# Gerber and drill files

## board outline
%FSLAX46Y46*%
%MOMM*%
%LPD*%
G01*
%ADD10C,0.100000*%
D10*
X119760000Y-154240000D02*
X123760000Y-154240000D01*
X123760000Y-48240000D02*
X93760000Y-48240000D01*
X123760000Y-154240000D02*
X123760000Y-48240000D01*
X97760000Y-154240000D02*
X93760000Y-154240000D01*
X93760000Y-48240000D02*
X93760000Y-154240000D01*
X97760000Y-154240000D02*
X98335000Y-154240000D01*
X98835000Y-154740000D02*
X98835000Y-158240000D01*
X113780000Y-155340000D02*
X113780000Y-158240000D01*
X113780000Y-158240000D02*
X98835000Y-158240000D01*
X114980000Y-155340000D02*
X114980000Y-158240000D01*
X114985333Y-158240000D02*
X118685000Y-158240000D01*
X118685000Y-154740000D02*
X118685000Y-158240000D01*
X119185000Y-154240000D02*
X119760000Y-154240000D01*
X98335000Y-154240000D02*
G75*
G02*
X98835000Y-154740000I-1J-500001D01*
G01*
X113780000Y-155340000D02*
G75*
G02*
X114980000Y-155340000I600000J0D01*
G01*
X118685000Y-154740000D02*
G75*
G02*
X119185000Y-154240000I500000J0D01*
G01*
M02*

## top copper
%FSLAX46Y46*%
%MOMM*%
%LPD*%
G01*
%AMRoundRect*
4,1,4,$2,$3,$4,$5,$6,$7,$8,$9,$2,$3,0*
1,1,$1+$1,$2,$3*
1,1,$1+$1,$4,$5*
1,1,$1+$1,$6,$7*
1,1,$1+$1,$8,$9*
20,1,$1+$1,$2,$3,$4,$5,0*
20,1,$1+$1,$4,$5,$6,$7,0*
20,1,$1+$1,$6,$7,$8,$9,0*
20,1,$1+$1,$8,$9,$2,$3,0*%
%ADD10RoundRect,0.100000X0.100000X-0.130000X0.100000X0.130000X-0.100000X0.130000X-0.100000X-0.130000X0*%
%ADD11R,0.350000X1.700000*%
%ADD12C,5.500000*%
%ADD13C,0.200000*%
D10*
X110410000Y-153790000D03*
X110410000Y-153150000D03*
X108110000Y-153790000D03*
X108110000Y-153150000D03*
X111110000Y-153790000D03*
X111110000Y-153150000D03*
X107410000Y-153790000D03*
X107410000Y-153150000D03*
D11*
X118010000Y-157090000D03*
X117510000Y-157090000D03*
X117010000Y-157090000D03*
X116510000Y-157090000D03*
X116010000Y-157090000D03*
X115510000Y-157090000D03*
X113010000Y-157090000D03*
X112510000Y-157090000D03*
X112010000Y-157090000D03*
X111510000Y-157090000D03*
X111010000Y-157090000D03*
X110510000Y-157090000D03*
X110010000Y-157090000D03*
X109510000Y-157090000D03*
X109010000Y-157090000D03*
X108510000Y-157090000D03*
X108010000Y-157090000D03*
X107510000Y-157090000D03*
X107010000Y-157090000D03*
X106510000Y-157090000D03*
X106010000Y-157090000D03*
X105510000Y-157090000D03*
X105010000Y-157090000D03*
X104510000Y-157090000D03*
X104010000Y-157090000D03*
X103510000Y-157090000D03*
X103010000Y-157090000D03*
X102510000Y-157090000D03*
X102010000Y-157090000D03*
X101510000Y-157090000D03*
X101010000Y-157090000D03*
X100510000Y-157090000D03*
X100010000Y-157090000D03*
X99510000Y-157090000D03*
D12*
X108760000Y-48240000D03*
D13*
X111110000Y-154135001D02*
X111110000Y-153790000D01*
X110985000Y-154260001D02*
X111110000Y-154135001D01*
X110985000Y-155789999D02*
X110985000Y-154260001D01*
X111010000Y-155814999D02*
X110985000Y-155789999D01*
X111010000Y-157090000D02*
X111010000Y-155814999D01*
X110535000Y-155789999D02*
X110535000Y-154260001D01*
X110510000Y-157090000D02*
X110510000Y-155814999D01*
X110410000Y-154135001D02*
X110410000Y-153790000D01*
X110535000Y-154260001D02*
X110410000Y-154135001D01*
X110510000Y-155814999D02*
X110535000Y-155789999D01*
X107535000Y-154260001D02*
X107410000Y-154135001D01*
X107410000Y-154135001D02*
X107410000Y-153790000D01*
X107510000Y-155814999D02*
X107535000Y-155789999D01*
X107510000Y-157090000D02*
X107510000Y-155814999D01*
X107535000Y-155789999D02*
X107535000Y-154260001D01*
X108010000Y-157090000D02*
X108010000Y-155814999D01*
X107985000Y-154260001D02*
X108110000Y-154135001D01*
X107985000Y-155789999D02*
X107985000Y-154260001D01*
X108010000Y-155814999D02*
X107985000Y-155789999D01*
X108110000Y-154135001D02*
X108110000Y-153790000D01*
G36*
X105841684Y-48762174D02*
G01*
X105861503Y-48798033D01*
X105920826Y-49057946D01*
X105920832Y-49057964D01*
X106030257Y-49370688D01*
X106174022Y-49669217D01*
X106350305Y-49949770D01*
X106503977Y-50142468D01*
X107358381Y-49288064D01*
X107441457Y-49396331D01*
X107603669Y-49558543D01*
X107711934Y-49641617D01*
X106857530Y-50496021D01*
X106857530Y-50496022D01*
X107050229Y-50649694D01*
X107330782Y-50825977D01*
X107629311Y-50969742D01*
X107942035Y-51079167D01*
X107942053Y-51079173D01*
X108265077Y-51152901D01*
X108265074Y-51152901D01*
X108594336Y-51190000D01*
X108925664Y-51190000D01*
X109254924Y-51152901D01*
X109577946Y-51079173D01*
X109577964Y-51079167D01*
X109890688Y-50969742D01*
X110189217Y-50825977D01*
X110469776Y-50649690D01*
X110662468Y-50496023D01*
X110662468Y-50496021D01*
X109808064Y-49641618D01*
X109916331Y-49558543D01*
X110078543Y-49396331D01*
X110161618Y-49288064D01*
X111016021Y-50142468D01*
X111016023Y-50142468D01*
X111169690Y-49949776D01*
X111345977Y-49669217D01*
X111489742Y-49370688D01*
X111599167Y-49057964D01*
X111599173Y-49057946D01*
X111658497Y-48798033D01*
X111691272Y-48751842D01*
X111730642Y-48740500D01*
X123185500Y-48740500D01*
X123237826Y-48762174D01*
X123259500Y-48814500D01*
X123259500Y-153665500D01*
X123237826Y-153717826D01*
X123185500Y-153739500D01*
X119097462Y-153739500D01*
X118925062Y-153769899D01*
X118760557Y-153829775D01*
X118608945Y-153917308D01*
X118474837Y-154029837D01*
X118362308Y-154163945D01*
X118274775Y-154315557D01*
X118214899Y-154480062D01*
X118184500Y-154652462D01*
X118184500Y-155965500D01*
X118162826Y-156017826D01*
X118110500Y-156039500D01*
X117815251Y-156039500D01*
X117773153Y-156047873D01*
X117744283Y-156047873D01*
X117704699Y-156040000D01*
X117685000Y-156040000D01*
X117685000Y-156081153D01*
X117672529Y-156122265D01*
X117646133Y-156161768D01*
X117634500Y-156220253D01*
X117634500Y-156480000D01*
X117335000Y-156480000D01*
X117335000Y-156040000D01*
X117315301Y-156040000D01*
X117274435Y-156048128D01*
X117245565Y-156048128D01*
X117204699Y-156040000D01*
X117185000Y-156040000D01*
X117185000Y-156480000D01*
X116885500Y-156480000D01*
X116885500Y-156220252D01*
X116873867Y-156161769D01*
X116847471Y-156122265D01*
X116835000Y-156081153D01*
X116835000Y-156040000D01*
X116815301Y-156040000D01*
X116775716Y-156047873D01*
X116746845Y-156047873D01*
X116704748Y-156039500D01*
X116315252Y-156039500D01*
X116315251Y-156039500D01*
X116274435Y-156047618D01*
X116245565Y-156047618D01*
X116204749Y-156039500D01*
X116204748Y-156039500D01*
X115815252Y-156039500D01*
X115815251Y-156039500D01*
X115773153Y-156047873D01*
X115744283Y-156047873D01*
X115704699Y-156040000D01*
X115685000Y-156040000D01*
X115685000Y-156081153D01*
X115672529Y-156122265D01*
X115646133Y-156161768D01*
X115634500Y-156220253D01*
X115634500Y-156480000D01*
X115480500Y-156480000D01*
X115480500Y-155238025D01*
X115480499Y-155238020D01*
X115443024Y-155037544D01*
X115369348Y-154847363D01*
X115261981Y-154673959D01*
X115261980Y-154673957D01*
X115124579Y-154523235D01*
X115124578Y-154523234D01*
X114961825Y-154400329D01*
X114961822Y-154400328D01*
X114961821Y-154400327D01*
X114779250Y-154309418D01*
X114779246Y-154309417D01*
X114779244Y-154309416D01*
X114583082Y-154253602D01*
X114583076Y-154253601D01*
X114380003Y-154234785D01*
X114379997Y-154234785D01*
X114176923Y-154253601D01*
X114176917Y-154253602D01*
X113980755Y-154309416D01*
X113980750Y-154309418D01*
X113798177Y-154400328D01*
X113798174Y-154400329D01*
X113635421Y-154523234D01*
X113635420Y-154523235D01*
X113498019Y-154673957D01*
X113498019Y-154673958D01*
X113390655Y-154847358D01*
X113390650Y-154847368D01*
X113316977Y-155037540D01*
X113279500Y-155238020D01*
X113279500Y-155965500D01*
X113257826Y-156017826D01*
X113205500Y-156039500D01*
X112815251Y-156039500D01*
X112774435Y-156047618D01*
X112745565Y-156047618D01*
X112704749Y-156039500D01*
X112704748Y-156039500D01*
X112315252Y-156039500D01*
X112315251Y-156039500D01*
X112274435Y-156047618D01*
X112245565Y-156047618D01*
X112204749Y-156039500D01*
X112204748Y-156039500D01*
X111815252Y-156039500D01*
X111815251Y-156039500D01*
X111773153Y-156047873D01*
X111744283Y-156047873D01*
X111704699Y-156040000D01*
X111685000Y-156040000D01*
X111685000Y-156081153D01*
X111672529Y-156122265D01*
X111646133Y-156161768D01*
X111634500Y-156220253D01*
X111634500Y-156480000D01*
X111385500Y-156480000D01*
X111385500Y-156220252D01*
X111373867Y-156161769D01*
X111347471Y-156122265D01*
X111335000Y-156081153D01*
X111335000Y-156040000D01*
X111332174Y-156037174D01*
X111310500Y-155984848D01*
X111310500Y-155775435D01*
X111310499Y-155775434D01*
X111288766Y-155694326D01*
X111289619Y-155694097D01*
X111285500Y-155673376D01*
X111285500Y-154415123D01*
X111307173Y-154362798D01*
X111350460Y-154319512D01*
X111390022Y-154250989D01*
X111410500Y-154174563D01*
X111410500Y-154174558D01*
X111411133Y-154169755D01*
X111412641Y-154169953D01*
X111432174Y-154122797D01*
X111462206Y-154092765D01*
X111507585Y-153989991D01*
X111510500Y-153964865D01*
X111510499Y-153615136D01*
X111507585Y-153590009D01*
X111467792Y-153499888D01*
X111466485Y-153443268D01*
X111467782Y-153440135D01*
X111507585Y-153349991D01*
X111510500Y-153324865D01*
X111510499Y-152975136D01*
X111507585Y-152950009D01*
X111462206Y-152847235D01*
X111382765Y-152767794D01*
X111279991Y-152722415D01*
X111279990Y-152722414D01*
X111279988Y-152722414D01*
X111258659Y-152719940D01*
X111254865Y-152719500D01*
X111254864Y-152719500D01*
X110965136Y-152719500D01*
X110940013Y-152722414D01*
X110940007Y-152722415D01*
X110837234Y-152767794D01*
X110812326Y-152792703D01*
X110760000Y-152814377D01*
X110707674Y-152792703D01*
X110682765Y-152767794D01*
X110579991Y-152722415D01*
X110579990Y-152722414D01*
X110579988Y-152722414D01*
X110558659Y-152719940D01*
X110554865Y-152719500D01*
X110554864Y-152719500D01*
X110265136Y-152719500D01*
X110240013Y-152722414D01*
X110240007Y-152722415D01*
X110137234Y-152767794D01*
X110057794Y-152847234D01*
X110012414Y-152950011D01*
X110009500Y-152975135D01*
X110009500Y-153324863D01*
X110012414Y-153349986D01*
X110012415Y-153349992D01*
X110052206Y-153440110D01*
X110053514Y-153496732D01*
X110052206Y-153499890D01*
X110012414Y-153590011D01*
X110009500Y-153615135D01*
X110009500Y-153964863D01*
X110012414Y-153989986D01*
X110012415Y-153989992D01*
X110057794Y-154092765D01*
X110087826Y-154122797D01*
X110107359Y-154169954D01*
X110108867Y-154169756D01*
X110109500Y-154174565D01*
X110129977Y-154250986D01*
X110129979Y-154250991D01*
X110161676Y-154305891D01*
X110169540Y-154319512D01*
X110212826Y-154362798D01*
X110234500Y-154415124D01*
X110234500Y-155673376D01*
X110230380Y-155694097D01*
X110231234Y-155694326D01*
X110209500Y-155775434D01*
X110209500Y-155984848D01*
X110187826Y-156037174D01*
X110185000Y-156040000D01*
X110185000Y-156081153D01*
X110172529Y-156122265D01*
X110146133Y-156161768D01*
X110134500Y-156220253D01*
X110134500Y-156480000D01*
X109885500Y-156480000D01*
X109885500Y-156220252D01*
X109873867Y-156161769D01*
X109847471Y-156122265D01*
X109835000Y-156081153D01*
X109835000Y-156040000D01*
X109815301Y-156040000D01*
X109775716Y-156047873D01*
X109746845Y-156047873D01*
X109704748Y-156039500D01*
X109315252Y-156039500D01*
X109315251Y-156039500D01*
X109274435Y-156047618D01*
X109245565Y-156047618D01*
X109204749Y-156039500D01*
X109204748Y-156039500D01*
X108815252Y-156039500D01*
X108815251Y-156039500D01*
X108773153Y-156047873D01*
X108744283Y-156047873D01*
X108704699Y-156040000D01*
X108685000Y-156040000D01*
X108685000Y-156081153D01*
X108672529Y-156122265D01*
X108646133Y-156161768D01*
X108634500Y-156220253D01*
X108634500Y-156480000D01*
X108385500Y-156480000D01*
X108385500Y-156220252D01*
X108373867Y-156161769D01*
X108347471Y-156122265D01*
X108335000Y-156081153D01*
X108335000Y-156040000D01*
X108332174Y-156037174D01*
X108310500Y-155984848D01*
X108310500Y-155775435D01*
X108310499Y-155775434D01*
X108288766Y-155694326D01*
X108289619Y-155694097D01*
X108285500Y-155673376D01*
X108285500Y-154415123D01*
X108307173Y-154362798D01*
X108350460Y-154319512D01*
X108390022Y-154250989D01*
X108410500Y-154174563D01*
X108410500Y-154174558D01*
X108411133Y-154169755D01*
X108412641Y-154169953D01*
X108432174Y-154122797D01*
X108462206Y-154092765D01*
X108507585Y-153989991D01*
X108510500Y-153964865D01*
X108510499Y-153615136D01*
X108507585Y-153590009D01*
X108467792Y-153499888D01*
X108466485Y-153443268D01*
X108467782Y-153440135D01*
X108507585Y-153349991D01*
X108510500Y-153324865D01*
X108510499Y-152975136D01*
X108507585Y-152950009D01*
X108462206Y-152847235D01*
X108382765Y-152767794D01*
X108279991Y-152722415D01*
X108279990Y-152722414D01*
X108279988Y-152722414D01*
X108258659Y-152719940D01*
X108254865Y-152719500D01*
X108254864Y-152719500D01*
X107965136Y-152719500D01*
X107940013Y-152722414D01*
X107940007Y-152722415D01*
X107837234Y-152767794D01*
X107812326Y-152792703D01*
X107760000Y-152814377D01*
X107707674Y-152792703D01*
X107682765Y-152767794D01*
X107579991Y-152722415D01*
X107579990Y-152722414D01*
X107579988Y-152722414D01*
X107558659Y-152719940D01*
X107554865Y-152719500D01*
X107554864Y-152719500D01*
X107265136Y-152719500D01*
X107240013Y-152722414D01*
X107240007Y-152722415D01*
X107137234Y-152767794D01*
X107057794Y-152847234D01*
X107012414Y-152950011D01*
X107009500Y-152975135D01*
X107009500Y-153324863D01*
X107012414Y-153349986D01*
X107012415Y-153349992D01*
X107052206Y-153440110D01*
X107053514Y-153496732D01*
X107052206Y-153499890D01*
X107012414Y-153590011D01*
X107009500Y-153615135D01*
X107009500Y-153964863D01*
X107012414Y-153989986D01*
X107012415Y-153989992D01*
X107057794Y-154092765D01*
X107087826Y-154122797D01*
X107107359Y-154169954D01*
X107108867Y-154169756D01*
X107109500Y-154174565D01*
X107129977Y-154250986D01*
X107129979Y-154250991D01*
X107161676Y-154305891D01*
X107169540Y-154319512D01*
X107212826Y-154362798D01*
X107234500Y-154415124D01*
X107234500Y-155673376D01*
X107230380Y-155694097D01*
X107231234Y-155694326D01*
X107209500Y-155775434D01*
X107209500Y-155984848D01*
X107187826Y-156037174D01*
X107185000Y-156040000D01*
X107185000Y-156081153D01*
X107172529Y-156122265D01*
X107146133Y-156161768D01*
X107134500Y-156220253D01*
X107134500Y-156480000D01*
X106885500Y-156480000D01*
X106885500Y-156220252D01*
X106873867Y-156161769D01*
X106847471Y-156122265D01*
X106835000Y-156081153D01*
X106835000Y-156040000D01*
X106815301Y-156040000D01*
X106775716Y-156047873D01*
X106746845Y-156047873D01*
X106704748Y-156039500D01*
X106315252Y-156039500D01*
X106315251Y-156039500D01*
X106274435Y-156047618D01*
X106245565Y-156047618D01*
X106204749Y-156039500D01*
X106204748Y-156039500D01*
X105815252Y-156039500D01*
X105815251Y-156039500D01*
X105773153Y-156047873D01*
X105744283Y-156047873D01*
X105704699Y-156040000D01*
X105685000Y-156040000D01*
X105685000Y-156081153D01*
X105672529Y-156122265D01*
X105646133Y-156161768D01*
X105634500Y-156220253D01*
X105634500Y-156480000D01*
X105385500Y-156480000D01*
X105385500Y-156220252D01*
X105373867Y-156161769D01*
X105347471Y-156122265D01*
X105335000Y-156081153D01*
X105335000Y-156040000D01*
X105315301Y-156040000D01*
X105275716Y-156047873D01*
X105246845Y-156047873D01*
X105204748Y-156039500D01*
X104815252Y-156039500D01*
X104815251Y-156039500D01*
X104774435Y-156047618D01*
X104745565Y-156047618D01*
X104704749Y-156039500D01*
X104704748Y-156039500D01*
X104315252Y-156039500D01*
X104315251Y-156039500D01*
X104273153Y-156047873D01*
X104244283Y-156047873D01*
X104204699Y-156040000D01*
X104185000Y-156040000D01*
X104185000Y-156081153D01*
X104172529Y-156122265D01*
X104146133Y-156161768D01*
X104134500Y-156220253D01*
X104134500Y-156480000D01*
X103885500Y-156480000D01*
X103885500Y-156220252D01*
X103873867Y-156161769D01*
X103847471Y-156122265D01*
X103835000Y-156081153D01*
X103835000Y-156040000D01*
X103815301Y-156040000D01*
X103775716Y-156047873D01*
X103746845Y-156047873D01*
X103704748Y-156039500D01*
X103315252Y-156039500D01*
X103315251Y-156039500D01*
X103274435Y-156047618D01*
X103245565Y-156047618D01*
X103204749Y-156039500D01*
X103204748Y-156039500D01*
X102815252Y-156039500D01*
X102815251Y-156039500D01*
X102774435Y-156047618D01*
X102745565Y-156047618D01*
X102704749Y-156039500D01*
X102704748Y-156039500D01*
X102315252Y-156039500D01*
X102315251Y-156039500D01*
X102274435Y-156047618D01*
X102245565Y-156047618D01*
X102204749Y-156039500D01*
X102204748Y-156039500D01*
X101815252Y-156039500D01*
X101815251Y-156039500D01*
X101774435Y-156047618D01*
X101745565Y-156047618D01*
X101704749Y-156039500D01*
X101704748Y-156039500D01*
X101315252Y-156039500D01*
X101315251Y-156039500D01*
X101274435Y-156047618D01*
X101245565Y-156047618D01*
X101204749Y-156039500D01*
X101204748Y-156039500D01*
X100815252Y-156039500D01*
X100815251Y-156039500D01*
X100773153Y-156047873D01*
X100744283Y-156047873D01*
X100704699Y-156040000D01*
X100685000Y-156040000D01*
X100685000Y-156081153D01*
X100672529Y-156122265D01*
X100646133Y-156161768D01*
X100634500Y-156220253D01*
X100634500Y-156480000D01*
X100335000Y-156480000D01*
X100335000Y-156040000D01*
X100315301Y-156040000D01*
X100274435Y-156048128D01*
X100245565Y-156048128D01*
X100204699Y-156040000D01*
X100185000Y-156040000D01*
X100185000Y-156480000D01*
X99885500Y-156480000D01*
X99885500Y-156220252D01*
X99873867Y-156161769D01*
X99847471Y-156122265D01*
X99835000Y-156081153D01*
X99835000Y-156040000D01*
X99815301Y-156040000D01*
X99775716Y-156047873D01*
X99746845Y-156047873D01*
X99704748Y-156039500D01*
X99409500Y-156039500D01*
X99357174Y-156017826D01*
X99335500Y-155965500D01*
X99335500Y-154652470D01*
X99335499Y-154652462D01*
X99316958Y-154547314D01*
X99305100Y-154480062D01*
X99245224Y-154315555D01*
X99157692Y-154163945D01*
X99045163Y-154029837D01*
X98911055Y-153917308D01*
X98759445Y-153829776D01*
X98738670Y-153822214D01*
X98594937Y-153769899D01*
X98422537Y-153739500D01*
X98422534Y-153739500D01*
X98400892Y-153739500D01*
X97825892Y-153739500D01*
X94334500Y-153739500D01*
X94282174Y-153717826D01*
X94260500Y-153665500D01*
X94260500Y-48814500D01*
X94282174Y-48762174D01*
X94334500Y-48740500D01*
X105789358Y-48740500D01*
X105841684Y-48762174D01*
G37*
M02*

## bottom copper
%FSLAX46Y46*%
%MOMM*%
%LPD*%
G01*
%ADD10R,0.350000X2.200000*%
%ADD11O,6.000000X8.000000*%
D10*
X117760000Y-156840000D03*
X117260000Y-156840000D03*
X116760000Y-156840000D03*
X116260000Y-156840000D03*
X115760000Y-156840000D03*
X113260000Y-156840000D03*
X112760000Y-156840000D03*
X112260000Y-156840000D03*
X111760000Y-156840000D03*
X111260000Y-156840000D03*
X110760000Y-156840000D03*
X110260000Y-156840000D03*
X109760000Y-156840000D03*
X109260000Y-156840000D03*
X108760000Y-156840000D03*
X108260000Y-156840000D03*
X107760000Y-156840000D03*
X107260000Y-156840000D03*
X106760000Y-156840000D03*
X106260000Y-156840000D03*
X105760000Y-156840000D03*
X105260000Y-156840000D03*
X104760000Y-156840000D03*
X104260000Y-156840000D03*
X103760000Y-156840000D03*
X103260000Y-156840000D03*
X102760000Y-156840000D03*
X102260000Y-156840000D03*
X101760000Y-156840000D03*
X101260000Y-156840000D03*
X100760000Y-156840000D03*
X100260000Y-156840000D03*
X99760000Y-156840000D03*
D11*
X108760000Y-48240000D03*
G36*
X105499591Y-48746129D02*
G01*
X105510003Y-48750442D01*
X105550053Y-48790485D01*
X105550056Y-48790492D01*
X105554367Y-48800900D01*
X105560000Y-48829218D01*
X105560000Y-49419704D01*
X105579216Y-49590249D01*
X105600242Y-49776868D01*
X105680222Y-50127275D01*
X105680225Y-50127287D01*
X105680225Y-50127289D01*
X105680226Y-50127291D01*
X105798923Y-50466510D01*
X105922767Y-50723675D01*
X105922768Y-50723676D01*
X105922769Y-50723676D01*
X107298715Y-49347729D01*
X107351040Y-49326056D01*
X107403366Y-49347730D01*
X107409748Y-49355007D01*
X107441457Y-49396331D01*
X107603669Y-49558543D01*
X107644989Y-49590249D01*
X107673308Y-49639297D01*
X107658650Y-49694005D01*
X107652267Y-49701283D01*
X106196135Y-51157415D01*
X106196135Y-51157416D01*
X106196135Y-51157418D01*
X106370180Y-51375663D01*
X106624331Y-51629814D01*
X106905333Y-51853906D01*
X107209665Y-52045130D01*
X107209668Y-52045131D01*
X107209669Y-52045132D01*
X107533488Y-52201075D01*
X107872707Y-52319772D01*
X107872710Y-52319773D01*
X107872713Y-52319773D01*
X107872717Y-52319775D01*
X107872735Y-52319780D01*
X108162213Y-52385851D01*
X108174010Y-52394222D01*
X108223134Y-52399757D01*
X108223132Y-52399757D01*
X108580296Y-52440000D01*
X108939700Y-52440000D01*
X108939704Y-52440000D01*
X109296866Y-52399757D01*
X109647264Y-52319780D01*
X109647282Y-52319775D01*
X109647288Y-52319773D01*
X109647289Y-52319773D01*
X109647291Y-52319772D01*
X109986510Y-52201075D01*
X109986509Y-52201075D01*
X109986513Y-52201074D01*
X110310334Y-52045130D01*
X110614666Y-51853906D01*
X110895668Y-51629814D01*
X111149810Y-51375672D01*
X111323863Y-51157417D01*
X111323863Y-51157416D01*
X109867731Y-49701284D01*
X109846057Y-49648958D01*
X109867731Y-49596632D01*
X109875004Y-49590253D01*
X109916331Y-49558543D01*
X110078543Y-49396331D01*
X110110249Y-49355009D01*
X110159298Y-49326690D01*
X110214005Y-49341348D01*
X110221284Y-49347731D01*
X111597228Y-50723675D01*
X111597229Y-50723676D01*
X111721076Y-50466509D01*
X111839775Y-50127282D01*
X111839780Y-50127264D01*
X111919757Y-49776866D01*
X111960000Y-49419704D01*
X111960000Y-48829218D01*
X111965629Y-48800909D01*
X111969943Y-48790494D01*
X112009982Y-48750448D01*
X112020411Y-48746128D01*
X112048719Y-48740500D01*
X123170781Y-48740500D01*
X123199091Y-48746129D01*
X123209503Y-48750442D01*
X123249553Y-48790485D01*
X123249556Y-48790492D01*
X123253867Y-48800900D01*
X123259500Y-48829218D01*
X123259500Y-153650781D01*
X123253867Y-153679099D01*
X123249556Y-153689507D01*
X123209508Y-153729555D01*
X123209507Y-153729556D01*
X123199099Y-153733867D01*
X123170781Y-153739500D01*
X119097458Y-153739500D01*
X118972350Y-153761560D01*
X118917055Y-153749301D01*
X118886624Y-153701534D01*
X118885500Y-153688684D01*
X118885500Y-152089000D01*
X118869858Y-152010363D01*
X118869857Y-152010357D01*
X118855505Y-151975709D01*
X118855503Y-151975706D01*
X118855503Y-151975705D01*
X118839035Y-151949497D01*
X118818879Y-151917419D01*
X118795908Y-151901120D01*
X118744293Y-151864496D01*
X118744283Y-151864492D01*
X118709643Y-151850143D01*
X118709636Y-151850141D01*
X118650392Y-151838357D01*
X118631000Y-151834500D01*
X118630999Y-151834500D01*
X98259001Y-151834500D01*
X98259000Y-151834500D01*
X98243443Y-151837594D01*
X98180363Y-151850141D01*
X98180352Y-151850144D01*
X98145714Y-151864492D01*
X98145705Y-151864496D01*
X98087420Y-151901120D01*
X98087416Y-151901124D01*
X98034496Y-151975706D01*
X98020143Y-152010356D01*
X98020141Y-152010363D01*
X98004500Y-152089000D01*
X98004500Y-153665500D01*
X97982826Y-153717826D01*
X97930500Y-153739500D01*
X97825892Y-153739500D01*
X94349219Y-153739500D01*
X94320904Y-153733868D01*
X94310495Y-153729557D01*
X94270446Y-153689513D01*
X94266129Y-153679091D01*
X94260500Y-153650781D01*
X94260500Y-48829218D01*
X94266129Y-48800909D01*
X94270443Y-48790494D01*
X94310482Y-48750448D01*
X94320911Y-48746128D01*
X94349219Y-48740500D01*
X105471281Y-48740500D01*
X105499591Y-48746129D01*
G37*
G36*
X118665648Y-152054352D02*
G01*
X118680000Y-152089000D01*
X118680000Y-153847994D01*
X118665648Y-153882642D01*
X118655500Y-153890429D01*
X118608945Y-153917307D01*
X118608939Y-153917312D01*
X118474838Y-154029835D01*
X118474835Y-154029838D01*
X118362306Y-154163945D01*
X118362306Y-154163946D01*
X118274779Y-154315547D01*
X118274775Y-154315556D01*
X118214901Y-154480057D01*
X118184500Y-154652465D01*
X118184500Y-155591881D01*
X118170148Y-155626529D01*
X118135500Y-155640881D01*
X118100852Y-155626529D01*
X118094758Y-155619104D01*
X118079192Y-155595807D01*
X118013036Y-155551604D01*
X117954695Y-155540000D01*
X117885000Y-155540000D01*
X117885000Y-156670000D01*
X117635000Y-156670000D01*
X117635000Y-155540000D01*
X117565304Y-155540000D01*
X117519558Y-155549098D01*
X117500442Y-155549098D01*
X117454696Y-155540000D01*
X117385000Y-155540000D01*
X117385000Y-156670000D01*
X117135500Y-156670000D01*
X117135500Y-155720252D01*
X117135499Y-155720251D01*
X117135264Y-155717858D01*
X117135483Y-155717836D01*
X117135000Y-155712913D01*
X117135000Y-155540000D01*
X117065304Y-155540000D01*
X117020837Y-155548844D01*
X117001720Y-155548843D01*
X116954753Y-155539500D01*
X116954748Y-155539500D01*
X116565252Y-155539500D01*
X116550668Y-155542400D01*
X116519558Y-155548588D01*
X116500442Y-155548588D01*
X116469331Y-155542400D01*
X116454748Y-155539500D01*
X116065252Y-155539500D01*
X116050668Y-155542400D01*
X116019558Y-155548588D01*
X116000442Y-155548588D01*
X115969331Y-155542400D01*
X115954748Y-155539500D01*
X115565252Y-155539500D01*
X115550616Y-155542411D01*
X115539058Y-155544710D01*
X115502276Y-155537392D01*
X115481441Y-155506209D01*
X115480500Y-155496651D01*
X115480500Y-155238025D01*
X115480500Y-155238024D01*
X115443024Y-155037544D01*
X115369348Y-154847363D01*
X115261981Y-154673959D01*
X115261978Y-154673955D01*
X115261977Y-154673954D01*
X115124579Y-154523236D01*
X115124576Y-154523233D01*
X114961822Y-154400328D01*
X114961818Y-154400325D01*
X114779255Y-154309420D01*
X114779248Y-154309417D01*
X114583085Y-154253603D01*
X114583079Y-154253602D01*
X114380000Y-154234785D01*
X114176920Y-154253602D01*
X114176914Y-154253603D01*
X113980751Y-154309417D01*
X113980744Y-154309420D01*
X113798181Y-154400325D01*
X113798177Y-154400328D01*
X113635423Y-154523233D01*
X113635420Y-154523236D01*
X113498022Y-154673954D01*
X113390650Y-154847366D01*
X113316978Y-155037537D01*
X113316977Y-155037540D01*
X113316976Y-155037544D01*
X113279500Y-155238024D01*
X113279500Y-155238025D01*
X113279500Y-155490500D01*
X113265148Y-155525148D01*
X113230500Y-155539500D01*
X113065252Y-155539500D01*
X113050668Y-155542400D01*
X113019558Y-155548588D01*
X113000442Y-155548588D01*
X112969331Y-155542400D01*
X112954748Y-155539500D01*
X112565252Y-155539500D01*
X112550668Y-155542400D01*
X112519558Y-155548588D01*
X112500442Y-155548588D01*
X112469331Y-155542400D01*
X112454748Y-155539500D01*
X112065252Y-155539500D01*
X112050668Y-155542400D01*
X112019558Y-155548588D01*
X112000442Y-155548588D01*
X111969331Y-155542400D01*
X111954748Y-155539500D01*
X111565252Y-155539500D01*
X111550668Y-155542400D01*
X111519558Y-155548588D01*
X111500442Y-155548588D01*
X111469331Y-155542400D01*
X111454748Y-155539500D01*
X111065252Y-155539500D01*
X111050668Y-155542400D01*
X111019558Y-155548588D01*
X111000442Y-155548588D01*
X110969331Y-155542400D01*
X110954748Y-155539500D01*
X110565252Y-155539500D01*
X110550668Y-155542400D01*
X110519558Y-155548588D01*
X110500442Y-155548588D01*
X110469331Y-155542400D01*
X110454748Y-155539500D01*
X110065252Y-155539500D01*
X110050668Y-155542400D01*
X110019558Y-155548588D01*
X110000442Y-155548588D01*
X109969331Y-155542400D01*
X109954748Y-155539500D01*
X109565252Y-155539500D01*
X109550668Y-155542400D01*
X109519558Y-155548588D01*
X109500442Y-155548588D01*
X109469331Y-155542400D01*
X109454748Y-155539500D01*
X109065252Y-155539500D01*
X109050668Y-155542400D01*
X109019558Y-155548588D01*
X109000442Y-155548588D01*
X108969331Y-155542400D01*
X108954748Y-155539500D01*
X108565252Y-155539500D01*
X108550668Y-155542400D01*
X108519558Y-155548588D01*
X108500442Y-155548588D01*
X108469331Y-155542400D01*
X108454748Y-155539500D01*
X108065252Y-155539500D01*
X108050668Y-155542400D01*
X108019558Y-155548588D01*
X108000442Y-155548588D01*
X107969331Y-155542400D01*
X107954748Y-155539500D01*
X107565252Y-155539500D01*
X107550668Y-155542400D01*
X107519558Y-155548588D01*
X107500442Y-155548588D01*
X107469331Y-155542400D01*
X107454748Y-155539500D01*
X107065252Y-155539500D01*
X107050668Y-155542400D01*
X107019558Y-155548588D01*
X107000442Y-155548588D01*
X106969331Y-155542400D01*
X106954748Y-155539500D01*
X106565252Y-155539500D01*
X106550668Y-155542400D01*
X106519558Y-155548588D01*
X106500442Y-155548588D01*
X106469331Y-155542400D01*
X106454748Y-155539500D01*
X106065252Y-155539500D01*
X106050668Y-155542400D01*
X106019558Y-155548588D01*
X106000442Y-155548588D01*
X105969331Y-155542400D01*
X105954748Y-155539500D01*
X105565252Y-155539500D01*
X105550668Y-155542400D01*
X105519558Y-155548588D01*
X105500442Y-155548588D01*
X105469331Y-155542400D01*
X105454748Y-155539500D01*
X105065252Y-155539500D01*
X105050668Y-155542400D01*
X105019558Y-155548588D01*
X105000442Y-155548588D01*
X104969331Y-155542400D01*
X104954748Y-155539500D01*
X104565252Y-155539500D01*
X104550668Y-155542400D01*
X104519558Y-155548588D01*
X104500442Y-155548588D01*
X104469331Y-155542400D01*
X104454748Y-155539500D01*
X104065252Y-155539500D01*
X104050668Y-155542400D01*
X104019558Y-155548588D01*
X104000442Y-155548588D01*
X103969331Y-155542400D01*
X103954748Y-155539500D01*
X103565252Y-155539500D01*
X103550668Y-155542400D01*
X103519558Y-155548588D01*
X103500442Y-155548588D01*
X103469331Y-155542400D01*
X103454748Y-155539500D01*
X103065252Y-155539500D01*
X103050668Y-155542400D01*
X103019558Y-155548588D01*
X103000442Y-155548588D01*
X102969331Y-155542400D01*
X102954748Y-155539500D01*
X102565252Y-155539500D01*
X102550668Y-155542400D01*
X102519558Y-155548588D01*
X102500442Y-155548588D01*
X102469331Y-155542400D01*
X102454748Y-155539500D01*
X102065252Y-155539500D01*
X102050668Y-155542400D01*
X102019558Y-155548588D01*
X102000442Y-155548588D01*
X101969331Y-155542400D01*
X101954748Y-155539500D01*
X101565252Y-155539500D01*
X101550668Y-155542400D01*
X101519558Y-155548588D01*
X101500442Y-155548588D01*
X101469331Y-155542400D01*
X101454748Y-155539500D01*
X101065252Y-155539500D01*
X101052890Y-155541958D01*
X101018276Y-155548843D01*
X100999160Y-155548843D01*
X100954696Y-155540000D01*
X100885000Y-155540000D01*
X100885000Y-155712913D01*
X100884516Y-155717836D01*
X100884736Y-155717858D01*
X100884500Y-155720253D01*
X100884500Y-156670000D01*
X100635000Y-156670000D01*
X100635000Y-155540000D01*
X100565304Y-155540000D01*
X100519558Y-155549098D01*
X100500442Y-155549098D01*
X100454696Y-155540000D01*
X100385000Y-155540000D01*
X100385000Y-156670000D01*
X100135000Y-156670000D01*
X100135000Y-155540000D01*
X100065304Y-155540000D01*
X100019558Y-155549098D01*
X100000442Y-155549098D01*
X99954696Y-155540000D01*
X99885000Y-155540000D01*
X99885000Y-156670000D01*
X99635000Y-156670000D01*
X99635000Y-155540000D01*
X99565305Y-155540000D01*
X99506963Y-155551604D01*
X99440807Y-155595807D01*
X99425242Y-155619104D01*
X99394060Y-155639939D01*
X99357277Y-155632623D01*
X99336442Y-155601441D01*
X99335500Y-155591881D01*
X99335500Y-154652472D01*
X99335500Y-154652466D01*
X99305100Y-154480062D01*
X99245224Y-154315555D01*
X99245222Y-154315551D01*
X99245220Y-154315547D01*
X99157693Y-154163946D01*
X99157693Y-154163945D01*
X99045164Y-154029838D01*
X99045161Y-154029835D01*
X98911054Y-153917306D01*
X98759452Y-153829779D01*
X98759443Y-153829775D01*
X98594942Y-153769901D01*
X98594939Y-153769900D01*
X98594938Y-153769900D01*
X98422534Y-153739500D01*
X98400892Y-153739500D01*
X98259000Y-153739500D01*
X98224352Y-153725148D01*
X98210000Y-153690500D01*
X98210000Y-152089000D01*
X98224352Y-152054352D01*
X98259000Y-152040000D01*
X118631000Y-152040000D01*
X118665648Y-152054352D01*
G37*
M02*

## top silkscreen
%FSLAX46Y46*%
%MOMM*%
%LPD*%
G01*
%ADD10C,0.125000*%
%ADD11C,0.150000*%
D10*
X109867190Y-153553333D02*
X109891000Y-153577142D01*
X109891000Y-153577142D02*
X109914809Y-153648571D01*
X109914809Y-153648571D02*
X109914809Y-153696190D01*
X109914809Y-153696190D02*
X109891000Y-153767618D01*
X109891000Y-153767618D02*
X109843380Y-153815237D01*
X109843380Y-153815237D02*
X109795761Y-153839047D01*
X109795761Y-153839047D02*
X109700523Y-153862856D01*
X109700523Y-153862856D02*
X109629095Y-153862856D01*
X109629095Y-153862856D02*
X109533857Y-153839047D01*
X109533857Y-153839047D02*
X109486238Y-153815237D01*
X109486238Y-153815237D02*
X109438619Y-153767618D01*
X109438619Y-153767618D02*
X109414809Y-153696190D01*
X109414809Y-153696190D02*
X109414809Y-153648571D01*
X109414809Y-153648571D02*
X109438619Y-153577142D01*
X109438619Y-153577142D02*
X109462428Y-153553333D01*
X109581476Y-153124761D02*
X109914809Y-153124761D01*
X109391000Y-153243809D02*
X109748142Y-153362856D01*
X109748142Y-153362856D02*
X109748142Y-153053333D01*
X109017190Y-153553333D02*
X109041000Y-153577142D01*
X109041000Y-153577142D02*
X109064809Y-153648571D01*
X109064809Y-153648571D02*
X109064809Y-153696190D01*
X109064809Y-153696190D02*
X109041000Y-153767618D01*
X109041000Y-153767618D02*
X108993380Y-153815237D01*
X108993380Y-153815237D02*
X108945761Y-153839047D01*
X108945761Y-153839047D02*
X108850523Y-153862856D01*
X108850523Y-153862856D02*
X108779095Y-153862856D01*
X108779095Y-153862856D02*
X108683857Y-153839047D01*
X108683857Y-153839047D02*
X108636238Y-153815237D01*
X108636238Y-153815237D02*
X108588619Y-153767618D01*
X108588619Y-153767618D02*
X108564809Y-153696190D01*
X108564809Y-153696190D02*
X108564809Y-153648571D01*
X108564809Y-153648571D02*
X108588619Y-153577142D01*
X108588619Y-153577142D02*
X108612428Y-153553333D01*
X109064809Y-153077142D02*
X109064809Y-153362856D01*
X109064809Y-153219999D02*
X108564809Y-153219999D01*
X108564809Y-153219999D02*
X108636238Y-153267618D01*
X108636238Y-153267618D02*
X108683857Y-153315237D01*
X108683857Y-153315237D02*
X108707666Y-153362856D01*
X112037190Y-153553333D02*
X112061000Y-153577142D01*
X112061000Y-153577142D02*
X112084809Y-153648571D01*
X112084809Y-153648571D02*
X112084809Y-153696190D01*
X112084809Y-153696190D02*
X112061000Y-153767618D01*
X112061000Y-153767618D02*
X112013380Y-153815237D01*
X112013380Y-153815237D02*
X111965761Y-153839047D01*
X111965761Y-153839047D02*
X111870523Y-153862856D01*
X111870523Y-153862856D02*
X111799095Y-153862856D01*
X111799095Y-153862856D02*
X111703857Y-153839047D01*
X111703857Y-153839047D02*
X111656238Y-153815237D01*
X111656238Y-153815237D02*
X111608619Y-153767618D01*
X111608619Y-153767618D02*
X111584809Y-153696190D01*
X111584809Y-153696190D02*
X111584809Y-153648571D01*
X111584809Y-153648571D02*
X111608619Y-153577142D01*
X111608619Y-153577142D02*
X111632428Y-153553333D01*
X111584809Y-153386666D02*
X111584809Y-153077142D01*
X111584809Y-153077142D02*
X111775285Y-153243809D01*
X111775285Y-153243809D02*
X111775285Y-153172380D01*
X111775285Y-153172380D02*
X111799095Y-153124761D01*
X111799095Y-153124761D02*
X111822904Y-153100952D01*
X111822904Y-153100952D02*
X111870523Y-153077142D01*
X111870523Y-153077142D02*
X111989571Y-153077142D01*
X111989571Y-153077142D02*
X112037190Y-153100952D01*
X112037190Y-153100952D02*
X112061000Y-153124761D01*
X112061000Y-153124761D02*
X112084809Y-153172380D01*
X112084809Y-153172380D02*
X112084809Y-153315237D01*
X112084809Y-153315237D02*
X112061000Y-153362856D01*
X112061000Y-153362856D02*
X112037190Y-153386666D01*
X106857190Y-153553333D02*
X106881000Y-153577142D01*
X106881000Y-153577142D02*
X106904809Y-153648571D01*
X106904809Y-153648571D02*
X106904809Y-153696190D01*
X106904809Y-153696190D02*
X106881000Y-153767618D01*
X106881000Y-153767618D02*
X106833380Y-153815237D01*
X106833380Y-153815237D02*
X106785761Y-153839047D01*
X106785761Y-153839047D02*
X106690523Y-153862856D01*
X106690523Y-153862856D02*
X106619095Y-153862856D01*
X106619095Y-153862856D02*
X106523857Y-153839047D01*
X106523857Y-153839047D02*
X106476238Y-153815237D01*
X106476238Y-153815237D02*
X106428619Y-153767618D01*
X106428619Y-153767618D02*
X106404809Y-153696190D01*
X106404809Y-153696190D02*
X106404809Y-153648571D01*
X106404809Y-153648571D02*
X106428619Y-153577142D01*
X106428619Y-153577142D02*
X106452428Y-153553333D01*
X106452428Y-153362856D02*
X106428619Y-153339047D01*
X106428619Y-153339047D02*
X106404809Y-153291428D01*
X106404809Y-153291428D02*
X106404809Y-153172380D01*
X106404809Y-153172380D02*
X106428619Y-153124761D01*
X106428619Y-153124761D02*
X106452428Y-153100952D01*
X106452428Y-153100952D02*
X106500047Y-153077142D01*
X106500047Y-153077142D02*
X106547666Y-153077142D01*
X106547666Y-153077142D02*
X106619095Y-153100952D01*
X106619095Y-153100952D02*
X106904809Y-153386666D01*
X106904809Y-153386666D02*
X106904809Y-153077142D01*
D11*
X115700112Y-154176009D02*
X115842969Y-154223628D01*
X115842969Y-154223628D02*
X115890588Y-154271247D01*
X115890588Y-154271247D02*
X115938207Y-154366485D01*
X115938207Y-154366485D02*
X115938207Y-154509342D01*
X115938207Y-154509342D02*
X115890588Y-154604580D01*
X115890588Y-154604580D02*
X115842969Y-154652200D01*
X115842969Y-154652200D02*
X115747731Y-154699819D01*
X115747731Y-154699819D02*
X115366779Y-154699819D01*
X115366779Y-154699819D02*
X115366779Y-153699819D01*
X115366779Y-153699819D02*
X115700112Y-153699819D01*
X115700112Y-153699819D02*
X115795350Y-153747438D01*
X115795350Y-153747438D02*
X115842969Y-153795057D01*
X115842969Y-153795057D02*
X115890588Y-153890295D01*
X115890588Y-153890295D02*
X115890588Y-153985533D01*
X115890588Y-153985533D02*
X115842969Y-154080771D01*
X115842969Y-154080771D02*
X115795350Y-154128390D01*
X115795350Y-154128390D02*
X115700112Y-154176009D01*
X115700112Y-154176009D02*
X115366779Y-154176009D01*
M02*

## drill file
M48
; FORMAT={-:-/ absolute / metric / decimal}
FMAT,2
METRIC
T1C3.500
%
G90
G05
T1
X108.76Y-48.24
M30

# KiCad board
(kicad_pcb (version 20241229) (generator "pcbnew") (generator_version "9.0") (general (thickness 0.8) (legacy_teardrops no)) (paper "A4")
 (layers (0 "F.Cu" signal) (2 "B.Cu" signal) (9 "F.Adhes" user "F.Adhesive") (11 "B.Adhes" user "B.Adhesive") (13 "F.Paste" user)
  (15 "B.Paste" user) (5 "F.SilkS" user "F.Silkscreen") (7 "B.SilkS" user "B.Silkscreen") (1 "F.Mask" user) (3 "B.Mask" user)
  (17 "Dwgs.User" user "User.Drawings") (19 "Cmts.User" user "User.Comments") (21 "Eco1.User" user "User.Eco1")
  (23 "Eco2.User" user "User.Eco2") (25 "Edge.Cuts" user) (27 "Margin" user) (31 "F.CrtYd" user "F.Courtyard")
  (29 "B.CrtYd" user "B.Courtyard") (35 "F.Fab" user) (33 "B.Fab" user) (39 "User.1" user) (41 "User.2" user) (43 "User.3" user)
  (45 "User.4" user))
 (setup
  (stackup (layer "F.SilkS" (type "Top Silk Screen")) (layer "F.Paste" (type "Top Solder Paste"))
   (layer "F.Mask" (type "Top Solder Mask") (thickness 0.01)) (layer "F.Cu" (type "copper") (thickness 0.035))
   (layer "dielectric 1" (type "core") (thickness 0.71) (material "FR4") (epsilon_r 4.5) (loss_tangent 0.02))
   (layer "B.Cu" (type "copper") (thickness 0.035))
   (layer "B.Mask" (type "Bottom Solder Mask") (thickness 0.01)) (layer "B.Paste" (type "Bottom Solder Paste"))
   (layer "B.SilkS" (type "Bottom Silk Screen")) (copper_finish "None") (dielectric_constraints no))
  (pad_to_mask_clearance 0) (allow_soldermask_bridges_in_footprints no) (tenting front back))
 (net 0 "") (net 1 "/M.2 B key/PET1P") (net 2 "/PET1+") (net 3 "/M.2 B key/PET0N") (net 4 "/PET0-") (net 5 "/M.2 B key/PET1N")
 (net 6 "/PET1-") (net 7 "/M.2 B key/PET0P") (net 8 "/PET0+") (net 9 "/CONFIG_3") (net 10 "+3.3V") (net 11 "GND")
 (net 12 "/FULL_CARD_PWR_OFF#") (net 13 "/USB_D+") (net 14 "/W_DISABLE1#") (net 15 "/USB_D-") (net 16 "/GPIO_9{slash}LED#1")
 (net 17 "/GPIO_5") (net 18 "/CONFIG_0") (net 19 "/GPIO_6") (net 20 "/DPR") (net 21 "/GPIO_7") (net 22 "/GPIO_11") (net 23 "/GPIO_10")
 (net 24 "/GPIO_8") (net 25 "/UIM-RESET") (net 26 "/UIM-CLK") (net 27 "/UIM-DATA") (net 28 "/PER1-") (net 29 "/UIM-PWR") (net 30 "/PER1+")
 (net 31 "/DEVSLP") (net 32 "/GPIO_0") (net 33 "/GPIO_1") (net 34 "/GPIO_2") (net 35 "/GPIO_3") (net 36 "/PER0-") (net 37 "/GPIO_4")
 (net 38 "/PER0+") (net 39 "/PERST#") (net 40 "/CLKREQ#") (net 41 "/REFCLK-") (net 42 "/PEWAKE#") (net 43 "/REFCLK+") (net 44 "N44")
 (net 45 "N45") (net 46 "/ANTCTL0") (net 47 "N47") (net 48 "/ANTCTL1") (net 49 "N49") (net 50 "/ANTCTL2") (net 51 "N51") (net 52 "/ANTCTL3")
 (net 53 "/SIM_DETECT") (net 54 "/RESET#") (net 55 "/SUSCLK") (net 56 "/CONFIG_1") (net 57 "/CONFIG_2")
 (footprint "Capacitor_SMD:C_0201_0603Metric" (layer "F.Cu") (at 110.41 153.47 90)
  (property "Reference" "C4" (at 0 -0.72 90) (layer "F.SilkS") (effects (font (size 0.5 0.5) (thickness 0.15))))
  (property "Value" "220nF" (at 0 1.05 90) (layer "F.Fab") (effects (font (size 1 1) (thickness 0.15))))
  (pad "" smd roundrect (at -0.345 0 90) (size 0.318 0.36) (layers "F.Paste") (roundrect_rratio 0.25))
  (pad "" smd roundrect (at 0.345 0 90) (size 0.318 0.36) (layers "F.Paste") (roundrect_rratio 0.25))
  (pad "1" smd roundrect (at -0.32 0 90) (size 0.46 0.4) (layers "F.Cu" "F.Mask") (roundrect_rratio 0.25) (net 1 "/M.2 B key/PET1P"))
  (pad "2" smd roundrect (at 0.32 0 90) (size 0.46 0.4) (layers "F.Cu" "F.Mask") (roundrect_rratio 0.25) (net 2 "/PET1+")))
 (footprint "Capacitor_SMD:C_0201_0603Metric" (layer "F.Cu") (at 108.11 153.47 90)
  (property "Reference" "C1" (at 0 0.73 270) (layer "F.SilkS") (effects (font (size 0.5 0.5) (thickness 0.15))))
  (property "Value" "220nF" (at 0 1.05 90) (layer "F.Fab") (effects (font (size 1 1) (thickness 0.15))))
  (pad "" smd roundrect (at -0.345 0 90) (size 0.318 0.36) (layers "F.Paste") (roundrect_rratio 0.25))
  (pad "" smd roundrect (at 0.345 0 90) (size 0.318 0.36) (layers "F.Paste") (roundrect_rratio 0.25))
  (pad "1" smd roundrect (at -0.32 0 90) (size 0.46 0.4) (layers "F.Cu" "F.Mask") (roundrect_rratio 0.25) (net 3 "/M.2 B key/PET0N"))
  (pad "2" smd roundrect (at 0.32 0 90) (size 0.46 0.4) (layers "F.Cu" "F.Mask") (roundrect_rratio 0.25) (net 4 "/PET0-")))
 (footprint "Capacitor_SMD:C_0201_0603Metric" (layer "F.Cu") (at 111.11 153.47 90)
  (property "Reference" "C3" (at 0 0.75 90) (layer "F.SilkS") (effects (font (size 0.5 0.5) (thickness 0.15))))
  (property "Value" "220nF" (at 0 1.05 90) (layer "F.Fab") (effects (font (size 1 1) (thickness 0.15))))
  (pad "" smd roundrect (at -0.345 0 90) (size 0.318 0.36) (layers "F.Paste") (roundrect_rratio 0.25))
  (pad "" smd roundrect (at 0.345 0 90) (size 0.318 0.36) (layers "F.Paste") (roundrect_rratio 0.25))
  (pad "1" smd roundrect (at -0.32 0 90) (size 0.46 0.4) (layers "F.Cu" "F.Mask") (roundrect_rratio 0.25) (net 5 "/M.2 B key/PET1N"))
  (pad "2" smd roundrect (at 0.32 0 90) (size 0.46 0.4) (layers "F.Cu" "F.Mask") (roundrect_rratio 0.25) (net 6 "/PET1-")))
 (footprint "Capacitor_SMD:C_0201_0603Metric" (layer "F.Cu") (at 107.41 153.47 90)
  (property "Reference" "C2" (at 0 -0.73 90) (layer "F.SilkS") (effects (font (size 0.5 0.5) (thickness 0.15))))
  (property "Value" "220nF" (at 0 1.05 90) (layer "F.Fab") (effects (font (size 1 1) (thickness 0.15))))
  (pad "" smd roundrect (at -0.345 0 90) (size 0.318 0.36) (layers "F.Paste") (roundrect_rratio 0.25))
  (pad "" smd roundrect (at 0.345 0 90) (size 0.318 0.36) (layers "F.Paste") (roundrect_rratio 0.25))
  (pad "1" smd roundrect (at -0.32 0 90) (size 0.46 0.4) (layers "F.Cu" "F.Mask") (roundrect_rratio 0.25) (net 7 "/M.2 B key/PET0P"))
  (pad "2" smd roundrect (at 0.32 0 90) (size 0.46 0.4) (layers "F.Cu" "F.Mask") (roundrect_rratio 0.25) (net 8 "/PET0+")))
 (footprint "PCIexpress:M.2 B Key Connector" (layer "F.Cu") (at 108.76 157.13)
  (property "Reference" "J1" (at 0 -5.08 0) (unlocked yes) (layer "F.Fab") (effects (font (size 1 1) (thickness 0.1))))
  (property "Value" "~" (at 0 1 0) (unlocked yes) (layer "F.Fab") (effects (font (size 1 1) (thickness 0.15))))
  (fp_line (start -11 -2.89) (end -10.425 -2.89) (stroke (width 0.1) (type default)) (layer "Edge.Cuts") (net 5))
  (fp_line (start -9.925 -2.39) (end -9.925 1.11) (stroke (width 0.1) (type default)) (layer "Edge.Cuts") (net 5))
  (fp_line (start 5.02 -1.79) (end 5.02 1.11) (stroke (width 0.1) (type default)) (layer "Edge.Cuts") (net 5))
  (fp_line (start 5.02 1.11) (end -9.925 1.11) (stroke (width 0.1) (type default)) (layer "Edge.Cuts") (net 5))
  (fp_line (start 6.22 -1.79) (end 6.22 1.11) (stroke (width 0.1) (type default)) (layer "Edge.Cuts") (net 5))
  (fp_line (start 6.225333 1.11) (end 9.925 1.11) (stroke (width 0.1) (type default)) (layer "Edge.Cuts") (net 5))
  (fp_line (start 9.925 -2.39) (end 9.925 1.11) (stroke (width 0.1) (type default)) (layer "Edge.Cuts") (net 5))
  (fp_line (start 10.425 -2.89) (end 11 -2.89) (stroke (width 0.1) (type default)) (layer "Edge.Cuts") (net 5))
  (fp_arc (start -10.425 -2.89) (mid -10.071447 -2.743553) (end -9.925 -2.39) (stroke (width 0.1) (type default)) (layer "Edge.Cuts")
   (net 5))
  (fp_arc (start 5.02 -1.79) (mid 5.62 -2.39) (end 6.22 -1.79) (stroke (width 0.1) (type default)) (layer "Edge.Cuts") (net 5))
  (fp_arc (start 9.925 -2.39) (mid 10.071447 -2.743553) (end 10.425 -2.89) (stroke (width 0.1) (type default)) (layer "Edge.Cuts") (net 5))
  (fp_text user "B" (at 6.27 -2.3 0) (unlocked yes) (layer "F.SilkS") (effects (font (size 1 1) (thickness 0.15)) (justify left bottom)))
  (pad "1" smd rect (at 9.25 -0.04 180) (size 0.35 1.7) (layers "F.Cu") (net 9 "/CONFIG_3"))
  (pad "2" smd rect (at 9 -0.29 180) (size 0.35 2.2) (layers "B.Cu") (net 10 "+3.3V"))
  (pad "3" smd rect (at 8.75 -0.04 180) (size 0.35 1.7) (layers "F.Cu") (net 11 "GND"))
  (pad "4" smd rect (at 8.5 -0.29 180) (size 0.35 2.2) (layers "B.Cu") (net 10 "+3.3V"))
  (pad "5" smd rect (at 8.25 -0.04 180) (size 0.35 1.7) (layers "F.Cu") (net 11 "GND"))
  (pad "6" smd rect (at 8 -0.29 180) (size 0.35 2.2) (layers "B.Cu") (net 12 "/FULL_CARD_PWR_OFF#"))
  (pad "7" smd rect (at 7.75 -0.04 180) (size 0.35 1.7) (layers "F.Cu") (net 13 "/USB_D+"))
  (pad "8" smd rect (at 7.5 -0.29 180) (size 0.35 2.2) (layers "B.Cu") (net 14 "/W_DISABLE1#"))
  (pad "9" smd rect (at 7.25 -0.04 180) (size 0.35 1.7) (layers "F.Cu") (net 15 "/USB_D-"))
  (pad "10" smd rect (at 7 -0.29 180) (size 0.35 2.2) (layers "B.Cu") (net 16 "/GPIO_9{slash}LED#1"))
  (pad "11" smd rect (at 6.75 -0.04 180) (size 0.35 1.7) (layers "F.Cu") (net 11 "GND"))
  (pad "20" smd rect (at 4.5 -0.29 180) (size 0.35 2.2) (layers "B.Cu") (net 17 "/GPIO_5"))
  (pad "21" smd rect (at 4.25 -0.04 180) (size 0.35 1.7) (layers "F.Cu") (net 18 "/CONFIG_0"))
  (pad "22" smd rect (at 4 -0.29 180) (size 0.35 2.2) (layers "B.Cu") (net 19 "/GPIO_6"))
  (pad "23" smd rect (at 3.75 -0.04 180) (size 0.35 1.7) (layers "F.Cu") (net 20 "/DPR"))
  (pad "24" smd rect (at 3.5 -0.29 180) (size 0.35 2.2) (layers "B.Cu") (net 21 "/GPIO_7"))
  (pad "25" smd rect (at 3.25 -0.04 180) (size 0.35 1.7) (layers "F.Cu") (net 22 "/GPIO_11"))
  (pad "26" smd rect (at 3 -0.29 180) (size 0.35 2.2) (layers "B.Cu") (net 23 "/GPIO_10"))
  (pad "27" smd rect (at 2.75 -0.04 180) (size 0.35 1.7) (layers "F.Cu") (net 11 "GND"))
  (pad "28" smd rect (at 2.5 -0.29 180) (size 0.35 2.2) (layers "B.Cu") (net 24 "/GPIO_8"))
  (pad "29" smd rect (at 2.25 -0.04 180) (size 0.35 1.7) (layers "F.Cu") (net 5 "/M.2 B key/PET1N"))
  (pad "30" smd rect (at 2 -0.29 180) (size 0.35 2.2) (layers "B.Cu") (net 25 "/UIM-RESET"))
  (pad "31" smd rect (at 1.75 -0.04 180) (size 0.35 1.7) (layers "F.Cu") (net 1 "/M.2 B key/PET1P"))
  (pad "32" smd rect (at 1.5 -0.29 180) (size 0.35 2.2) (layers "B.Cu") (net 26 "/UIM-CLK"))
  (pad "33" smd rect (at 1.25 -0.04 180) (size 0.35 1.7) (layers "F.Cu") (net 11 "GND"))
  (pad "34" smd rect (at 1 -0.29 180) (size 0.35 2.2) (layers "B.Cu") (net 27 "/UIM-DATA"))
  (pad "35" smd rect (at 0.75 -0.04 180) (size 0.35 1.7) (layers "F.Cu") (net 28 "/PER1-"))
  (pad "36" smd rect (at 0.5 -0.29 180) (size 0.35 2.2) (layers "B.Cu") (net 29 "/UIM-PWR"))
  (pad "37" smd rect (at 0.25 -0.04 180) (size 0.35 1.7) (layers "F.Cu") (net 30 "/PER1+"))
  (pad "38" smd rect (at 0 -0.29 180) (size 0.35 2.2) (layers "B.Cu") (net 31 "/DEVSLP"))
  (pad "39" smd rect (at -0.25 -0.04 180) (size 0.35 1.7) (layers "F.Cu") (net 11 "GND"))
  (pad "40" smd rect (at -0.5 -0.29 180) (size 0.35 2.2) (layers "B.Cu") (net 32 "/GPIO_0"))
  (pad "41" smd rect (at -0.75 -0.04 180) (size 0.35 1.7) (layers "F.Cu") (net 3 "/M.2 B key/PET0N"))
  (pad "42" smd rect (at -1 -0.29 180) (size 0.35 2.2) (layers "B.Cu") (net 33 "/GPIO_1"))
  (pad "43" smd rect (at -1.25 -0.04 180) (size 0.35 1.7) (layers "F.Cu") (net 7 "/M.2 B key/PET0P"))
  (pad "44" smd rect (at -1.5 -0.29 180) (size 0.35 2.2) (layers "B.Cu") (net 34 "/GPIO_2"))
  (pad "45" smd rect (at -1.75 -0.04 180) (size 0.35 1.7) (layers "F.Cu") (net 11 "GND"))
  (pad "46" smd rect (at -2 -0.29 180) (size 0.35 2.2) (layers "B.Cu") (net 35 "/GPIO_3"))
  (pad "47" smd rect (at -2.25 -0.04 180) (size 0.35 1.7) (layers "F.Cu") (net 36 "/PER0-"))
  (pad "48" smd rect (at -2.5 -0.29 180) (size 0.35 2.2) (layers "B.Cu") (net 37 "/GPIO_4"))
  (pad "49" smd rect (at -2.75 -0.04 180) (size 0.35 1.7) (layers "F.Cu") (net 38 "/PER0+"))
  (pad "50" smd rect (at -3 -0.29 180) (size 0.35 2.2) (layers "B.Cu") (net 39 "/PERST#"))
  (pad "51" smd rect (at -3.25 -0.04 180) (size 0.35 1.7) (layers "F.Cu") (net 11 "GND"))
  (pad "52" smd rect (at -3.5 -0.29 180) (size 0.35 2.2) (layers "B.Cu") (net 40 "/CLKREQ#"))
  (pad "53" smd rect (at -3.75 -0.04 180) (size 0.35 1.7) (layers "F.Cu") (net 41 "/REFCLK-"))
  (pad "54" smd rect (at -4 -0.29 180) (size 0.35 2.2) (layers "B.Cu") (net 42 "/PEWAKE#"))
  (pad "55" smd rect (at -4.25 -0.04 180) (size 0.35 1.7) (layers "F.Cu") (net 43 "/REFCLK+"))
  (pad "56" smd rect (at -4.5 -0.29 180) (size 0.35 2.2) (layers "B.Cu") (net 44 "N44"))
  (pad "57" smd rect (at -4.75 -0.04 180) (size 0.35 1.7) (layers "F.Cu") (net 11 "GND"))
  (pad "58" smd rect (at -5 -0.29 180) (size 0.35 2.2) (layers "B.Cu") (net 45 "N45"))
  (pad "59" smd rect (at -5.25 -0.04 180) (size 0.35 1.7) (layers "F.Cu") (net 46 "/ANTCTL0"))
  (pad "60" smd rect (at -5.5 -0.29 180) (size 0.35 2.2) (layers "B.Cu") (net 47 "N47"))
  (pad "61" smd rect (at -5.75 -0.04 180) (size 0.35 1.7) (layers "F.Cu") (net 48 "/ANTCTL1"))
  (pad "62" smd rect (at -6 -0.29 180) (size 0.35 2.2) (layers "B.Cu") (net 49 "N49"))
  (pad "63" smd rect (at -6.25 -0.04 180) (size 0.35 1.7) (layers "F.Cu") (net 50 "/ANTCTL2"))
  (pad "64" smd rect (at -6.5 -0.29 180) (size 0.35 2.2) (layers "B.Cu") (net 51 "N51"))
  (pad "65" smd rect (at -6.75 -0.04 180) (size 0.35 1.7) (layers "F.Cu") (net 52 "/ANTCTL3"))
  (pad "66" smd rect (at -7 -0.29 180) (size 0.35 2.2) (layers "B.Cu") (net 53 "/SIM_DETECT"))
  (pad "67" smd rect (at -7.25 -0.04 180) (size 0.35 1.7) (layers "F.Cu") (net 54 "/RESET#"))
  (pad "68" smd rect (at -7.5 -0.29 180) (size 0.35 2.2) (layers "B.Cu") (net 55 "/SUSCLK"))
  (pad "69" smd rect (at -7.75 -0.04 180) (size 0.35 1.7) (layers "F.Cu") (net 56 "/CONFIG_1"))
  (pad "70" smd rect (at -8 -0.29 180) (size 0.35 2.2) (layers "B.Cu") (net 10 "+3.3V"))
  (pad "71" smd rect (at -8.25 -0.04 180) (size 0.35 1.7) (layers "F.Cu") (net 11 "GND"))
  (pad "72" smd rect (at -8.5 -0.29 180) (size 0.35 2.2) (layers "B.Cu") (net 10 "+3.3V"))
  (pad "73" smd rect (at -8.75 -0.04 180) (size 0.35 1.7) (layers "F.Cu") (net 11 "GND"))
  (pad "74" smd rect (at -9 -0.29 180) (size 0.35 2.2) (layers "B.Cu") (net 10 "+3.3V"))
  (pad "75" smd rect (at -9.25 -0.04 180) (size 0.35 1.7) (layers "F.Cu") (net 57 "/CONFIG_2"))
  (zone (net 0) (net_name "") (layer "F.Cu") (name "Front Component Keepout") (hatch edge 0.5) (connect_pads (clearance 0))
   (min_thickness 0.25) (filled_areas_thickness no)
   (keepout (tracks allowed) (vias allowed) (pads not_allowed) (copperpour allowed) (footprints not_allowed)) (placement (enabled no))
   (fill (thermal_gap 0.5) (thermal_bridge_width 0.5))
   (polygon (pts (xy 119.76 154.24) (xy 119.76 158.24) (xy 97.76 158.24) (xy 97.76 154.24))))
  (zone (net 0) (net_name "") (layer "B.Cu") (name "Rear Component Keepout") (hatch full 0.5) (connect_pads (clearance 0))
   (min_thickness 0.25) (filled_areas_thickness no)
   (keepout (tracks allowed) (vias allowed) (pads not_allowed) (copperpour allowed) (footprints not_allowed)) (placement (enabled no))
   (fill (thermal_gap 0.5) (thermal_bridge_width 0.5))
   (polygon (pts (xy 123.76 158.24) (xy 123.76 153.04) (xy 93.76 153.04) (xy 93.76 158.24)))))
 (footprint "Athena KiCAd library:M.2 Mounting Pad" (layer "F.Cu") (at 108.76 48.24)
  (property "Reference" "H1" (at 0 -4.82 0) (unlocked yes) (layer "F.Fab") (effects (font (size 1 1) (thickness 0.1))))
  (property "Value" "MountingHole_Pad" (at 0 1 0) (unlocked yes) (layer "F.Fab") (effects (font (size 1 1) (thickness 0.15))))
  (pad "1" thru_hole circle (at 0 0) (size 5.5 5.5) (drill 3.5) (layers "*.Cu" "*.Mask") (remove_unused_layers no) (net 11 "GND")
   (padstack (mode front_inner_back)
    (layer "Inner" (shape circle) (size 5.5 5.5) (zone_connect -1))
    (layer "B.Cu" (shape oval) (size 6 8) (thermal_bridge_angle 45) (zone_connect -1)))))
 (gr_line (start 119.76 154.24) (end 123.76 154.24) (stroke (width 0.1) (type default)) (layer "Edge.Cuts"))
 (gr_line (start 123.76 48.24) (end 93.76 48.24) (stroke (width 0.1) (type default)) (layer "Edge.Cuts"))
 (gr_line (start 123.76 154.24) (end 123.76 48.24) (stroke (width 0.1) (type default)) (layer "Edge.Cuts"))
 (gr_line (start 97.76 154.24) (end 93.76 154.24) (stroke (width 0.1) (type default)) (layer "Edge.Cuts"))
 (gr_line (start 93.76 48.24) (end 93.76 154.24) (stroke (width 0.1) (type default)) (layer "Edge.Cuts"))
 (segment (start 111.11 154.135001) (end 111.11 153.79) (width 0.2) (layer "F.Cu") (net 5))
 (segment (start 110.985 154.260001) (end 111.11 154.135001) (width 0.2) (layer "F.Cu") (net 5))
 (segment (start 110.985 155.789999) (end 110.985 154.260001) (width 0.2) (layer "F.Cu") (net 5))
 (segment (start 111.01 155.814999) (end 110.985 155.789999) (width 0.2) (layer "F.Cu") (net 5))
 (segment (start 111.01 157.09) (end 111.01 155.814999) (width 0.2) (layer "F.Cu") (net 5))
 (segment (start 110.535 155.789999) (end 110.535 154.260001) (width 0.2) (layer "F.Cu") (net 1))
 (segment (start 110.51 157.09) (end 110.51 155.814999) (width 0.2) (layer "F.Cu") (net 1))
 (segment (start 110.41 154.135001) (end 110.41 153.79) (width 0.2) (layer "F.Cu") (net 1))
 (segment (start 110.535 154.260001) (end 110.41 154.135001) (width 0.2) (layer "F.Cu") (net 1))
 (segment (start 110.51 155.814999) (end 110.535 155.789999) (width 0.2) (layer "F.Cu") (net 1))
 (segment (start 107.535 154.260001) (end 107.41 154.135001) (width 0.2) (layer "F.Cu") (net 7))
 (segment (start 107.41 154.135001) (end 107.41 153.79) (width 0.2) (layer "F.Cu") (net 7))
 (segment (start 107.51 155.814999) (end 107.535 155.789999) (width 0.2) (layer "F.Cu") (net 7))
 (segment (start 107.51 157.09) (end 107.51 155.814999) (width 0.2) (layer "F.Cu") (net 7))
 (segment (start 107.535 155.789999) (end 107.535 154.260001) (width 0.2) (layer "F.Cu") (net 7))
 (segment (start 108.01 157.09) (end 108.01 155.814999) (width 0.2) (layer "F.Cu") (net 3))
 (segment (start 107.985 154.260001) (end 108.11 154.135001) (width 0.2) (layer "F.Cu") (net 3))
 (segment (start 107.985 155.789999) (end 107.985 154.260001) (width 0.2) (layer "F.Cu") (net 3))
 (segment (start 108.01 155.814999) (end 107.985 155.789999) (width 0.2) (layer "F.Cu") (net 3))
 (segment (start 108.11 154.135001) (end 108.11 153.79) (width 0.2) (layer "F.Cu") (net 3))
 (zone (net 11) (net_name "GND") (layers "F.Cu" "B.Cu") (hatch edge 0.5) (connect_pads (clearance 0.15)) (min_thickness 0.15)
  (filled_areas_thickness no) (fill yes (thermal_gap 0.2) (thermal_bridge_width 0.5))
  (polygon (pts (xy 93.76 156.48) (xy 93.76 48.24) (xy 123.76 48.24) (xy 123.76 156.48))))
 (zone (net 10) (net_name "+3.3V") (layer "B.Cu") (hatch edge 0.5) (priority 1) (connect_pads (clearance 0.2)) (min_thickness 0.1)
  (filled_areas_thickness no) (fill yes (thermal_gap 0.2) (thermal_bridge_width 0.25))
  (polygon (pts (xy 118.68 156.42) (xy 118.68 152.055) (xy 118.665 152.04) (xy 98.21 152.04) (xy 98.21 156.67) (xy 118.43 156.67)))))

